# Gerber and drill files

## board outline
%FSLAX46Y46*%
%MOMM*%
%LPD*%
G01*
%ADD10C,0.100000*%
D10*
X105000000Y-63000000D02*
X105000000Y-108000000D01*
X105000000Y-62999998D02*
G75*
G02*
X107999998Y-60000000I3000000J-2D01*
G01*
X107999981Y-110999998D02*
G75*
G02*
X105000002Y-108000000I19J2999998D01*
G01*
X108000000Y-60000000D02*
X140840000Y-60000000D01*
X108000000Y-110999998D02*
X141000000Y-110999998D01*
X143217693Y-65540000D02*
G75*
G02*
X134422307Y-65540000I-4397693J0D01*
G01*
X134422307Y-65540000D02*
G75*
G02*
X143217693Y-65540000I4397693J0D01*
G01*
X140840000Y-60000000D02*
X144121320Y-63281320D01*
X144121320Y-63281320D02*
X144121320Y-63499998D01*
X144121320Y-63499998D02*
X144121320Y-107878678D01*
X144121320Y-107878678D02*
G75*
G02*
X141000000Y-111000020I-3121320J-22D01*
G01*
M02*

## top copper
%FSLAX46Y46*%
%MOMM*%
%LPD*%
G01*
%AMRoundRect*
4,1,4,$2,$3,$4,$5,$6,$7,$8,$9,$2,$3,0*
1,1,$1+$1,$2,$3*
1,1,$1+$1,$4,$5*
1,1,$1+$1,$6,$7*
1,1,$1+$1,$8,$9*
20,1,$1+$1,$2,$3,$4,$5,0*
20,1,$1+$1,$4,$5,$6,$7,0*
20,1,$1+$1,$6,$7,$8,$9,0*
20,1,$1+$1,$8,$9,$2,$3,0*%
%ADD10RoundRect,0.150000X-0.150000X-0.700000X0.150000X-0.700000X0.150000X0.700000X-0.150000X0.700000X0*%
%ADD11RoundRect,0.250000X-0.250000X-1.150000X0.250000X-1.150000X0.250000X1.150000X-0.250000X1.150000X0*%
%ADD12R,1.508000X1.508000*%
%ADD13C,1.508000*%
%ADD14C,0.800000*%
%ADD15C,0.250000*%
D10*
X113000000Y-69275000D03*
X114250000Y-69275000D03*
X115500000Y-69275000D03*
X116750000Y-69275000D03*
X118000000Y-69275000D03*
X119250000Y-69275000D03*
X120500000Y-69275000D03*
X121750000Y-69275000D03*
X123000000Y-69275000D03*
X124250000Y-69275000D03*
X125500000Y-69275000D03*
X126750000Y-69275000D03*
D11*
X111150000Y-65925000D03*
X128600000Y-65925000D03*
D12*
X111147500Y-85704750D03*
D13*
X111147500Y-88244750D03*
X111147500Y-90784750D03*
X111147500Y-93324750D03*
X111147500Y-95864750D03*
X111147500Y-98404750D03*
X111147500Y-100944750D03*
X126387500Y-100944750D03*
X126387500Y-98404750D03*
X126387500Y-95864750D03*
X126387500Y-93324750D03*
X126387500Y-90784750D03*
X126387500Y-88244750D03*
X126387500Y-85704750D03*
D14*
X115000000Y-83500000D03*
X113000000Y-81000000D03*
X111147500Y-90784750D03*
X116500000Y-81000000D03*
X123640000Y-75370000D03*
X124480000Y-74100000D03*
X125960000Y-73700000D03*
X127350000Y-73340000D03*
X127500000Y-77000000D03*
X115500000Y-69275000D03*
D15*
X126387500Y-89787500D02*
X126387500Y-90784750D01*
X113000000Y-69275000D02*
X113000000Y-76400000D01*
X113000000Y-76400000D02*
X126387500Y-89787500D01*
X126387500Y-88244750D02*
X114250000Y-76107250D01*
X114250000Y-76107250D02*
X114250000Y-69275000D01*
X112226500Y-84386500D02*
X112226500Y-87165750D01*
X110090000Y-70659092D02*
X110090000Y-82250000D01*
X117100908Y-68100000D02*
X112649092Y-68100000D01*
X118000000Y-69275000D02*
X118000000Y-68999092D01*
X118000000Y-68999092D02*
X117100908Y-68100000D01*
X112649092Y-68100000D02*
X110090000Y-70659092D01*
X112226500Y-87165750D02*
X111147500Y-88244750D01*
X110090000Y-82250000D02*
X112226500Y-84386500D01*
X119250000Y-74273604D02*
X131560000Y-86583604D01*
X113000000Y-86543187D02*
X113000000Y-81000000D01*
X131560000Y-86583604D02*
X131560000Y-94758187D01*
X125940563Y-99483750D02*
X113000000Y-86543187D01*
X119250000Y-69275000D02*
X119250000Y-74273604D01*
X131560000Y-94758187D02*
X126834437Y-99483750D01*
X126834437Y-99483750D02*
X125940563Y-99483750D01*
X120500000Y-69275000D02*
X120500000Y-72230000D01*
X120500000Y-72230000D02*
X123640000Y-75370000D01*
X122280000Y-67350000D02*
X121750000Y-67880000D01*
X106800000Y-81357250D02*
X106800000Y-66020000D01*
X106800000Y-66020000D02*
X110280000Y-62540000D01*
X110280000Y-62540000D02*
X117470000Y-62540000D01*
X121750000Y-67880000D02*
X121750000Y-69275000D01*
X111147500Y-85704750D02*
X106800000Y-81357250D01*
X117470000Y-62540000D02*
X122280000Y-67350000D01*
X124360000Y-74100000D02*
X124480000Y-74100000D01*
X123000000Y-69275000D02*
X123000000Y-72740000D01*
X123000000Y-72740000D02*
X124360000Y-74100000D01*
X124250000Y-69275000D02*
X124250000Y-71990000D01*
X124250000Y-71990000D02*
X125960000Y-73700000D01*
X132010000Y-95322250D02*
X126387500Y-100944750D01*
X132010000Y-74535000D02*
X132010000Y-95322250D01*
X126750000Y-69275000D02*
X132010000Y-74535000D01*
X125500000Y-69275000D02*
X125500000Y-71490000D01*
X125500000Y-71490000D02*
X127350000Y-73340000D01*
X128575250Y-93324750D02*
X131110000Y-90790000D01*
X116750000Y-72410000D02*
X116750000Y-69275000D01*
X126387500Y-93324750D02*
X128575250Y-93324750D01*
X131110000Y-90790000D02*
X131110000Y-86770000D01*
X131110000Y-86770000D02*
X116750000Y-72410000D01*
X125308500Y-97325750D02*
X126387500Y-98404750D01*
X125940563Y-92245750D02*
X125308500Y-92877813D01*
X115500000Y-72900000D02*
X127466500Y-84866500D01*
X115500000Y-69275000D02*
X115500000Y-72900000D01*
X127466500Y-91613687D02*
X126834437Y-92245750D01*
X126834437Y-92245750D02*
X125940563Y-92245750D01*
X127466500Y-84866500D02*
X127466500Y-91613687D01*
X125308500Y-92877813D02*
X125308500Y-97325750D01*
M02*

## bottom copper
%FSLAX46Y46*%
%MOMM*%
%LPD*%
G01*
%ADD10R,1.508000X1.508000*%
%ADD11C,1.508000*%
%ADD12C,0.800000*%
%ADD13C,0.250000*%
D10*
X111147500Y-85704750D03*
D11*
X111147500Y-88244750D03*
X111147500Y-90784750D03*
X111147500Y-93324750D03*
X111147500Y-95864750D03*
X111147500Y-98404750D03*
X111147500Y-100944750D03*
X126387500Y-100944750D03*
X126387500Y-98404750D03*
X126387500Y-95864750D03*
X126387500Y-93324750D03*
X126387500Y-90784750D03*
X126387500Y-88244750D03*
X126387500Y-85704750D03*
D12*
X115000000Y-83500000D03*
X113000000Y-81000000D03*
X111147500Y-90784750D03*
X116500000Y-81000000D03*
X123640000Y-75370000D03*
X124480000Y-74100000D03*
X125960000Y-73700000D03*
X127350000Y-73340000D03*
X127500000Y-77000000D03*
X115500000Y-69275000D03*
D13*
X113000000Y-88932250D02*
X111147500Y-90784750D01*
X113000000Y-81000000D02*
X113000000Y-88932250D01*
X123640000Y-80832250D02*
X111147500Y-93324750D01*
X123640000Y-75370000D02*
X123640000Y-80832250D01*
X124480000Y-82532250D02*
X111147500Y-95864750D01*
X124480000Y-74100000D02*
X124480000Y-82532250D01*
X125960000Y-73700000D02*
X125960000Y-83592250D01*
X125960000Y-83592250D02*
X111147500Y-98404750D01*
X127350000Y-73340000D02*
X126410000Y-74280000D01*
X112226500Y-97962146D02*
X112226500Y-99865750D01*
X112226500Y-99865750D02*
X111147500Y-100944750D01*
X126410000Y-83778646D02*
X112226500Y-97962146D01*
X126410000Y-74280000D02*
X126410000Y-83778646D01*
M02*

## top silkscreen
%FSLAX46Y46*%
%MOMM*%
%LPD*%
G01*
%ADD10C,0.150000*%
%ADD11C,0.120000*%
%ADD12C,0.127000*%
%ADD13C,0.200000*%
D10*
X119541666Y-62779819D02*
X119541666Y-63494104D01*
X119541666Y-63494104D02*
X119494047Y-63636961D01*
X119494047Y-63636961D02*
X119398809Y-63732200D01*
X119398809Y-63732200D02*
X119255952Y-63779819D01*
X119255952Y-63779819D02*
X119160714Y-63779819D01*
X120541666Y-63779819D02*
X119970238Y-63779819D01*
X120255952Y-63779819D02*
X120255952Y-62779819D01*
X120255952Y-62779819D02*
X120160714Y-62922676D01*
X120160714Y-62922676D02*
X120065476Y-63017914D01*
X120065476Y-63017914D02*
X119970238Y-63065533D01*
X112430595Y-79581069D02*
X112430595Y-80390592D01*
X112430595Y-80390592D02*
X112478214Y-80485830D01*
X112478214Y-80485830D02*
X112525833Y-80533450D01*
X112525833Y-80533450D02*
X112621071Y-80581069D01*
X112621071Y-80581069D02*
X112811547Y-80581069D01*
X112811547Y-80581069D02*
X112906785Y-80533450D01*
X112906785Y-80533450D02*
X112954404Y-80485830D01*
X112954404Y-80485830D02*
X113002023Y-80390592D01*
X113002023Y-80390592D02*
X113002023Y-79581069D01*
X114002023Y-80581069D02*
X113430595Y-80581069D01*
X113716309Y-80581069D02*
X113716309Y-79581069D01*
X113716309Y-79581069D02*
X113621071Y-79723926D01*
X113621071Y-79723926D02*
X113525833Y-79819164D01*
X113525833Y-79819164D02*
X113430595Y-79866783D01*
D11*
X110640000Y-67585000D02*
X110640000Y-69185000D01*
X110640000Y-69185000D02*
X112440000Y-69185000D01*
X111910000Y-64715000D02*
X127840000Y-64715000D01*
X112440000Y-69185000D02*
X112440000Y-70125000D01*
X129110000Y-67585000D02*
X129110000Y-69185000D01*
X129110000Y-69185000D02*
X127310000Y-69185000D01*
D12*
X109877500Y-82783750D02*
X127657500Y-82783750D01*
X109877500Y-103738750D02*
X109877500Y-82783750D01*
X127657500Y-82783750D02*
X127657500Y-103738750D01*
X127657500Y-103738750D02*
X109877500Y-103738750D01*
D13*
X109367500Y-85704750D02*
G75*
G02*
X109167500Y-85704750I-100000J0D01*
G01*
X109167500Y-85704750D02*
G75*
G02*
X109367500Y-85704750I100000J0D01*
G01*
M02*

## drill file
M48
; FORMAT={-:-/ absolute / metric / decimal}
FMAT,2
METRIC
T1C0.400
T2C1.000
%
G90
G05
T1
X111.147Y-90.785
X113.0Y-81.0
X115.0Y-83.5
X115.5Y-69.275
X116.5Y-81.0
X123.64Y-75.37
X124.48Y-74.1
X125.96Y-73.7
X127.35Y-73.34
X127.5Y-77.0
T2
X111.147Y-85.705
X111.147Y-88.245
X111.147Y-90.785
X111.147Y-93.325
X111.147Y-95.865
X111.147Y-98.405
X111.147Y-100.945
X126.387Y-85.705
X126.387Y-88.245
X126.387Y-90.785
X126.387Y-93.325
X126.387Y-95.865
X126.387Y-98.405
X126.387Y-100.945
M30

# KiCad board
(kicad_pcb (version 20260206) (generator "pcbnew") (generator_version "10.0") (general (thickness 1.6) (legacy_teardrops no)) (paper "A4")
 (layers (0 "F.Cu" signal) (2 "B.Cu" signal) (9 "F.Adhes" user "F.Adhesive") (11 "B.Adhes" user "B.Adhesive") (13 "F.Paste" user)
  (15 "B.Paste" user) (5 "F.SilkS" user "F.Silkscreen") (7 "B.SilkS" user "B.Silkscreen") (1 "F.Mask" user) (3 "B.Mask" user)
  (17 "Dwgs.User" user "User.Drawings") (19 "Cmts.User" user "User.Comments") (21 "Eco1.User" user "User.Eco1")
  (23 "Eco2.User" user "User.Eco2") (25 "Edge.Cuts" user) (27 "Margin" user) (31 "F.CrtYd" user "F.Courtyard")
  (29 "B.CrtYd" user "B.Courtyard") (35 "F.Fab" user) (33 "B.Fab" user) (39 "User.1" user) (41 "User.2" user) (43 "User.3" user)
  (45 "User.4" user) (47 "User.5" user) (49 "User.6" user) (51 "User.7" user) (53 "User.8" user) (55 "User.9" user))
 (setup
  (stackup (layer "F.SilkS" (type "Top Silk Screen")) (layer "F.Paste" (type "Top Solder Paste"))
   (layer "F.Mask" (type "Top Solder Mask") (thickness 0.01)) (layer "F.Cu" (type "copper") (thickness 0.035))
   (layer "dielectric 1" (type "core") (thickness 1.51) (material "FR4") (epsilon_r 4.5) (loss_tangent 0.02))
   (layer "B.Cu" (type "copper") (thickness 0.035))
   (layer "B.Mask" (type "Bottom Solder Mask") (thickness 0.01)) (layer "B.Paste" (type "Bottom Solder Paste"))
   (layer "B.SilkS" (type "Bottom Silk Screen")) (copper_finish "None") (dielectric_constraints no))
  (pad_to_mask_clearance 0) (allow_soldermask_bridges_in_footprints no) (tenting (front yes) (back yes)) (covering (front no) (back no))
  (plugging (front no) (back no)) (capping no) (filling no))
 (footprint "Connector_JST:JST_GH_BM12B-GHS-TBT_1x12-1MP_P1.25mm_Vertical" (layer "F.Cu") (at 119.875 67.325)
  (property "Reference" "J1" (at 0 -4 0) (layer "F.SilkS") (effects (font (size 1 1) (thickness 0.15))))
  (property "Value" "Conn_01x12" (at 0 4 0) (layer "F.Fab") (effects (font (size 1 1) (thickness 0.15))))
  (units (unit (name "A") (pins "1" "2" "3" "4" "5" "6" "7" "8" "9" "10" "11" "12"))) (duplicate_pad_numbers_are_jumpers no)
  (fp_line (start -9.235 0.26) (end -9.235 1.86) (stroke (width 0.12) (type solid)) (layer "F.SilkS"))
  (fp_line (start -9.235 1.86) (end -7.435 1.86) (stroke (width 0.12) (type solid)) (layer "F.SilkS"))
  (fp_line (start -7.965 -2.61) (end 7.965 -2.61) (stroke (width 0.12) (type solid)) (layer "F.SilkS"))
  (fp_line (start -7.435 1.86) (end -7.435 2.8) (stroke (width 0.12) (type solid)) (layer "F.SilkS"))
  (fp_line (start 9.235 0.26) (end 9.235 1.86) (stroke (width 0.12) (type solid)) (layer "F.SilkS"))
  (fp_line (start 9.235 1.86) (end 7.435 1.86) (stroke (width 0.12) (type solid)) (layer "F.SilkS"))
  (pad "1" smd roundrect (at -6.875 1.95) (size 0.6 1.7) (layers "F.Cu" "F.Mask" "F.Paste") (roundrect_rratio 0.25) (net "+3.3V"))
  (pad "2" smd roundrect (at -5.625 1.95) (size 0.6 1.7) (layers "F.Cu" "F.Mask" "F.Paste") (roundrect_rratio 0.25) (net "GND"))
  (pad "3" smd roundrect (at -4.375 1.95) (size 0.6 1.7) (layers "F.Cu" "F.Mask" "F.Paste") (roundrect_rratio 0.25) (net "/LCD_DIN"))
  (pad "4" smd roundrect (at -3.125 1.95) (size 0.6 1.7) (layers "F.Cu" "F.Mask" "F.Paste") (roundrect_rratio 0.25) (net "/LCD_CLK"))
  (pad "5" smd roundrect (at -1.875 1.95) (size 0.6 1.7) (layers "F.Cu" "F.Mask" "F.Paste") (roundrect_rratio 0.25) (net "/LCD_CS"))
  (pad "6" smd roundrect (at -0.625 1.95) (size 0.6 1.7) (layers "F.Cu" "F.Mask" "F.Paste") (roundrect_rratio 0.25) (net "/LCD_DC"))
  (pad "7" smd roundrect (at 0.625 1.95) (size 0.6 1.7) (layers "F.Cu" "F.Mask" "F.Paste") (roundrect_rratio 0.25) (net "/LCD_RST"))
  (pad "8" smd roundrect (at 1.875 1.95) (size 0.6 1.7) (layers "F.Cu" "F.Mask" "F.Paste") (roundrect_rratio 0.25) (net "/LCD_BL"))
  (pad "9" smd roundrect (at 3.125 1.95) (size 0.6 1.7) (layers "F.Cu" "F.Mask" "F.Paste") (roundrect_rratio 0.25) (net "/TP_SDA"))
  (pad "10" smd roundrect (at 4.375 1.95) (size 0.6 1.7) (layers "F.Cu" "F.Mask" "F.Paste") (roundrect_rratio 0.25) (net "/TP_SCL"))
  (pad "11" smd roundrect (at 5.625 1.95) (size 0.6 1.7) (layers "F.Cu" "F.Mask" "F.Paste") (roundrect_rratio 0.25) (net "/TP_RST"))
  (pad "12" smd roundrect (at 6.875 1.95) (size 0.6 1.7) (layers "F.Cu" "F.Mask" "F.Paste") (roundrect_rratio 0.25) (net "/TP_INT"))
  (pad "MP" smd roundrect (at -8.725 -1.4) (size 1 2.8) (layers "F.Cu" "F.Mask" "F.Paste") (roundrect_rratio 0.25))
  (pad "MP" smd roundrect (at 8.725 -1.4) (size 1 2.8) (layers "F.Cu" "F.Mask" "F.Paste") (roundrect_rratio 0.25)))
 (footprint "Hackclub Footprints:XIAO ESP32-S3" (layer "F.Cu") (at 118.7675 93.26125)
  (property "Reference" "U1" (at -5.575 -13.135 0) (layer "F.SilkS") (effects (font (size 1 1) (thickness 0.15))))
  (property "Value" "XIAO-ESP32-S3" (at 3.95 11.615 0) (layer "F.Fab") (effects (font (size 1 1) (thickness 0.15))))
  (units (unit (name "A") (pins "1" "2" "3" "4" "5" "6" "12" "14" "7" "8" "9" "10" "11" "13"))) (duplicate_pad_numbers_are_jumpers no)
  (fp_line (start -8.89 -10.4775) (end 8.89 -10.4775) (stroke (width 0.127) (type solid)) (layer "F.SilkS"))
  (fp_line (start -8.89 10.4775) (end -8.89 -10.4775) (stroke (width 0.127) (type solid)) (layer "F.SilkS"))
  (fp_line (start 8.89 -10.4775) (end 8.89 10.4775) (stroke (width 0.127) (type solid)) (layer "F.SilkS"))
  (fp_line (start 8.89 10.4775) (end -8.89 10.4775) (stroke (width 0.127) (type solid)) (layer "F.SilkS"))
  (fp_circle (center -9.5 -7.5565) (end -9.4 -7.5565) (stroke (width 0.2) (type solid)) (fill no) (layer "F.SilkS"))
  (pad "1" thru_hole rect (at -7.62 -7.5565) (size 1.508 1.508) (drill 1) (layers "*.Cu" "*.Mask") (remove_unused_layers no) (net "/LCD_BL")
   (solder_mask_margin 0.102))
  (pad "2" thru_hole circle (at -7.62 -5.0165) (size 1.508 1.508) (drill 1) (layers "*.Cu" "*.Mask") (remove_unused_layers no)
   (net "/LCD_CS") (solder_mask_margin 0.102))
  (pad "3" thru_hole circle (at -7.62 -2.4765) (size 1.508 1.508) (drill 1) (layers "*.Cu" "*.Mask") (remove_unused_layers no)
   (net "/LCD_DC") (solder_mask_margin 0.102))
  (pad "4" thru_hole circle (at -7.62 0.0635) (size 1.508 1.508) (drill 1) (layers "*.Cu" "*.Mask") (remove_unused_layers no)
   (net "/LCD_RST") (solder_mask_margin 0.102))
  (pad "5" thru_hole circle (at -7.62 2.6035) (size 1.508 1.508) (drill 1) (layers "*.Cu" "*.Mask") (remove_unused_layers no)
   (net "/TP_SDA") (solder_mask_margin 0.102))
  (pad "6" thru_hole circle (at -7.62 5.1435) (size 1.508 1.508) (drill 1) (layers "*.Cu" "*.Mask") (remove_unused_layers no)
   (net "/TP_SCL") (solder_mask_margin 0.102))
  (pad "7" thru_hole circle (at -7.62 7.6835) (size 1.508 1.508) (drill 1) (layers "*.Cu" "*.Mask") (remove_unused_layers no)
   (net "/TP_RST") (solder_mask_margin 0.102))
  (pad "8" thru_hole circle (at 7.62 7.6835) (size 1.508 1.508) (drill 1) (layers "*.Cu" "*.Mask") (remove_unused_layers no) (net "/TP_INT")
   (solder_mask_margin 0.102))
  (pad "9" thru_hole circle (at 7.62 5.1435) (size 1.508 1.508) (drill 1) (layers "*.Cu" "*.Mask") (remove_unused_layers no)
   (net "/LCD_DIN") (solder_mask_margin 0.102))
  (pad "10" thru_hole circle (at 7.62 2.6035) (size 1.508 1.508) (drill 1) (layers "*.Cu" "*.Mask") (remove_unused_layers no)
   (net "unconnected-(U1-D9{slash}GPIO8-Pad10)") (solder_mask_margin 0.102))
  (pad "11" thru_hole circle (at 7.62 0.0635) (size 1.508 1.508) (drill 1) (layers "*.Cu" "*.Mask") (remove_unused_layers no)
   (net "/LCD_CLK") (solder_mask_margin 0.102))
  (pad "12" thru_hole circle (at 7.62 -2.4765) (size 1.508 1.508) (drill 1) (layers "*.Cu" "*.Mask") (remove_unused_layers no) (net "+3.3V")
   (solder_mask_margin 0.102))
  (pad "13" thru_hole circle (at 7.62 -5.0165) (size 1.508 1.508) (drill 1) (layers "*.Cu" "*.Mask") (remove_unused_layers no) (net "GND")
   (solder_mask_margin 0.102))
  (pad "14" thru_hole circle (at 7.62 -7.5565) (size 1.508 1.508) (drill 1) (layers "*.Cu" "*.Mask") (remove_unused_layers no)
   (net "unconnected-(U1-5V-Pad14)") (solder_mask_margin 0.102)))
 (gr_line (start 105 63) (end 105 108) (stroke (width 0.1) (type default)) (layer "Edge.Cuts"))
 (gr_arc (start 105 62.999998) (mid 105.878679 60.878679) (end 107.999998 60) (stroke (width 0.1) (type default)) (layer "Edge.Cuts"))
 (gr_arc (start 107.999981 110.999998) (mid 105.878661 110.121319) (end 104.999982 108) (stroke (width 0.1) (type default))
  (layer "Edge.Cuts"))
 (gr_line (start 108 60) (end 140.84 60) (stroke (width 0.1) (type default)) (layer "Edge.Cuts"))
 (gr_line (start 108 110.999998) (end 141 110.999998) (stroke (width 0.1) (type default)) (layer "Edge.Cuts"))
 (gr_circle (center 138.82 65.54) (end 141.36 69.13) (stroke (width 0.1) (type default)) (fill no) (layer "Edge.Cuts"))
 (gr_line (start 140.84 60) (end 144.12132 63.28132) (stroke (width 0.1) (type default)) (layer "Edge.Cuts"))
 (gr_line (start 144.12132 63.28132) (end 144.12132 63.499998) (stroke (width 0.1) (type default)) (layer "Edge.Cuts"))
 (gr_line (start 144.12132 63.499998) (end 144.12132 107.878678) (stroke (width 0.1) (type default)) (layer "Edge.Cuts"))
 (gr_arc (start 144.12132 107.878678) (mid 143.207107 110.085785) (end 141 110.999998) (stroke (width 0.1) (type default))
  (layer "Edge.Cuts"))
 (segment (start 126.3875 89.7875) (end 126.3875 90.78475) (width 0.25) (layer "F.Cu") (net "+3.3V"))
 (segment (start 113 69.275) (end 113 76.4) (width 0.25) (layer "F.Cu") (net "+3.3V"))
 (segment (start 113 76.4) (end 126.3875 89.7875) (width 0.25) (layer "F.Cu") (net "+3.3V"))
 (segment (start 126.3875 88.24475) (end 114.25 76.10725) (width 0.25) (layer "F.Cu") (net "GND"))
 (segment (start 114.25 76.10725) (end 114.25 69.275) (width 0.25) (layer "F.Cu") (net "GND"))
 (segment (start 112.2265 84.3865) (end 112.2265 87.16575) (width 0.25) (layer "F.Cu") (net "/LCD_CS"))
 (segment (start 110.09 70.659092) (end 110.09 82.25) (width 0.25) (layer "F.Cu") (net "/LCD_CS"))
 (segment (start 117.100908 68.1) (end 112.649092 68.1) (width 0.25) (layer "F.Cu") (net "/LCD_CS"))
 (segment (start 118 69.275) (end 118 68.999092) (width 0.25) (layer "F.Cu") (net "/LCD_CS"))
 (segment (start 118 68.999092) (end 117.100908 68.1) (width 0.25) (layer "F.Cu") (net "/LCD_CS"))
 (segment (start 112.649092 68.1) (end 110.09 70.659092) (width 0.25) (layer "F.Cu") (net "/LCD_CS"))
 (segment (start 112.2265 87.16575) (end 111.1475 88.24475) (width 0.25) (layer "F.Cu") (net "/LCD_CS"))
 (segment (start 110.09 82.25) (end 112.2265 84.3865) (width 0.25) (layer "F.Cu") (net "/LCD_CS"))
 (via (at 115 83.5) (size 0.8) (drill 0.4) (layers "F.Cu" "B.Cu") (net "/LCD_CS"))
 (segment (start 119.25 74.273604) (end 131.56 86.583604) (width 0.25) (layer "F.Cu") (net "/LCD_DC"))
 (segment (start 113 86.543187) (end 113 81) (width 0.25) (layer "F.Cu") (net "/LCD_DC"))
 (segment (start 131.56 86.583604) (end 131.56 94.758187) (width 0.25) (layer "F.Cu") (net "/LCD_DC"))
 (segment (start 125.940563 99.48375) (end 113 86.543187) (width 0.25) (layer "F.Cu") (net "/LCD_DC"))
 (segment (start 119.25 69.275) (end 119.25 74.273604) (width 0.25) (layer "F.Cu") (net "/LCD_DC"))
 (segment (start 131.56 94.758187) (end 126.834437 99.48375) (width 0.25) (layer "F.Cu") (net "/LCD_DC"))
 (segment (start 126.834437 99.48375) (end 125.940563 99.48375) (width 0.25) (layer "F.Cu") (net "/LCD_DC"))
 (via (at 113 81) (size 0.8) (drill 0.4) (layers "F.Cu" "B.Cu") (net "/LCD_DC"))
 (via (at 111.1475 90.78475) (size 0.8) (drill 0.4) (layers "F.Cu" "B.Cu") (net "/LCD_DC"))
 (segment (start 113 88.93225) (end 111.1475 90.78475) (width 0.25) (layer "B.Cu") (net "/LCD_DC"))
 (segment (start 113 81) (end 113 88.93225) (width 0.25) (layer "B.Cu") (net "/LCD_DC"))
 (segment (start 120.5 69.275) (end 120.5 72.23) (width 0.25) (layer "F.Cu") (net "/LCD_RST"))
 (segment (start 120.5 72.23) (end 123.64 75.37) (width 0.25) (layer "F.Cu") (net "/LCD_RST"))
 (via (at 116.5 81) (size 0.8) (drill 0.4) (layers "F.Cu" "B.Cu") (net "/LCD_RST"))
 (via (at 123.64 75.37) (size 0.8) (drill 0.4) (layers "F.Cu" "B.Cu") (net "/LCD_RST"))
 (segment (start 123.64 80.83225) (end 111.1475 93.32475) (width 0.25) (layer "B.Cu") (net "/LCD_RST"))
 (segment (start 123.64 75.37) (end 123.64 80.83225) (width 0.25) (layer "B.Cu") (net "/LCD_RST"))
 (segment (start 122.28 67.35) (end 121.75 67.88) (width 0.25) (layer "F.Cu") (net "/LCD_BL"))
 (segment (start 106.8 81.35725) (end 106.8 66.02) (width 0.25) (layer "F.Cu") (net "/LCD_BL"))
 (segment (start 106.8 66.02) (end 110.28 62.54) (width 0.25) (layer "F.Cu") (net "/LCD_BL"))
 (segment (start 110.28 62.54) (end 117.47 62.54) (width 0.25) (layer "F.Cu") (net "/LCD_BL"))
 (segment (start 121.75 67.88) (end 121.75 69.275) (width 0.25) (layer "F.Cu") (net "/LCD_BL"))
 (segment (start 111.1475 85.70475) (end 106.8 81.35725) (width 0.25) (layer "F.Cu") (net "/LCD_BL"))
 (segment (start 117.47 62.54) (end 122.28 67.35) (width 0.25) (layer "F.Cu") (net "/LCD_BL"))
 (segment (start 124.36 74.1) (end 124.48 74.1) (width 0.25) (layer "F.Cu") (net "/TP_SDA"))
 (segment (start 123 69.275) (end 123 72.74) (width 0.25) (layer "F.Cu") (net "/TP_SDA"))
 (segment (start 123 72.74) (end 124.36 74.1) (width 0.25) (layer "F.Cu") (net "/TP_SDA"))
 (via (at 124.48 74.1) (size 0.8) (drill 0.4) (layers "F.Cu" "B.Cu") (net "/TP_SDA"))
 (segment (start 124.48 82.53225) (end 111.1475 95.86475) (width 0.25) (layer "B.Cu") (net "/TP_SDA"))
 (segment (start 124.48 74.1) (end 124.48 82.53225) (width 0.25) (layer "B.Cu") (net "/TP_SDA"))
 (segment (start 124.25 69.275) (end 124.25 71.99) (width 0.25) (layer "F.Cu") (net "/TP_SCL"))
 (segment (start 124.25 71.99) (end 125.96 73.7) (width 0.25) (layer "F.Cu") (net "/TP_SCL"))
 (via (at 125.96 73.7) (size 0.8) (drill 0.4) (layers "F.Cu" "B.Cu") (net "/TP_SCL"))
 (segment (start 125.96 73.7) (end 125.96 83.59225) (width 0.25) (layer "B.Cu") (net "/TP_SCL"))
 (segment (start 125.96 83.59225) (end 111.1475 98.40475) (width 0.25) (layer "B.Cu") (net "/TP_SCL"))
 (segment (start 132.01 95.32225) (end 126.3875 100.94475) (width 0.25) (layer "F.Cu") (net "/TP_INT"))
 (segment (start 132.01 74.535) (end 132.01 95.32225) (width 0.25) (layer "F.Cu") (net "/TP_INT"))
 (segment (start 126.75 69.275) (end 132.01 74.535) (width 0.25) (layer "F.Cu") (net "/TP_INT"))
 (segment (start 125.5 69.275) (end 125.5 71.49) (width 0.25) (layer "F.Cu") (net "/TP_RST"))
 (segment (start 125.5 71.49) (end 127.35 73.34) (width 0.25) (layer "F.Cu") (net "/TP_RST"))
 (via (at 127.35 73.34) (size 0.8) (drill 0.4) (layers "F.Cu" "B.Cu") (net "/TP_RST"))
 (segment (start 127.35 73.34) (end 126.41 74.28) (width 0.25) (layer "B.Cu") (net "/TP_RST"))
 (segment (start 112.2265 97.962146) (end 112.2265 99.86575) (width 0.25) (layer "B.Cu") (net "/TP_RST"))
 (segment (start 112.2265 99.86575) (end 111.1475 100.94475) (width 0.25) (layer "B.Cu") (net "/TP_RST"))
 (segment (start 126.41 83.778646) (end 112.2265 97.962146) (width 0.25) (layer "B.Cu") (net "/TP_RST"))
 (segment (start 126.41 74.28) (end 126.41 83.778646) (width 0.25) (layer "B.Cu") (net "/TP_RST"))
 (segment (start 128.57525 93.32475) (end 131.11 90.79) (width 0.25) (layer "F.Cu") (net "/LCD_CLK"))
 (segment (start 116.75 72.41) (end 116.75 69.275) (width 0.25) (layer "F.Cu") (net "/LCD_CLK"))
 (segment (start 126.3875 93.32475) (end 128.57525 93.32475) (width 0.25) (layer "F.Cu") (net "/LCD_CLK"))
 (segment (start 131.11 90.79) (end 131.11 86.77) (width 0.25) (layer "F.Cu") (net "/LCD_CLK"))
 (segment (start 131.11 86.77) (end 116.75 72.41) (width 0.25) (layer "F.Cu") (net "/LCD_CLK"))
 (segment (start 125.3085 97.32575) (end 126.3875 98.40475) (width 0.25) (layer "F.Cu") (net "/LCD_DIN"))
 (segment (start 125.940563 92.24575) (end 125.3085 92.877813) (width 0.25) (layer "F.Cu") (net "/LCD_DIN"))
 (segment (start 115.5 72.9) (end 127.4665 84.8665) (width 0.25) (layer "F.Cu") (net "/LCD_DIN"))
 (segment (start 115.5 69.275) (end 115.5 72.9) (width 0.25) (layer "F.Cu") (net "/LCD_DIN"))
 (segment (start 127.4665 91.613687) (end 126.834437 92.24575) (width 0.25) (layer "F.Cu") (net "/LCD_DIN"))
 (segment (start 126.834437 92.24575) (end 125.940563 92.24575) (width 0.25) (layer "F.Cu") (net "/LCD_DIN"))
 (segment (start 127.4665 84.8665) (end 127.4665 91.613687) (width 0.25) (layer "F.Cu") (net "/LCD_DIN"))
 (segment (start 125.3085 92.877813) (end 125.3085 97.32575) (width 0.25) (layer "F.Cu") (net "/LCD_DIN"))
 (via (at 127.5 77) (size 0.8) (drill 0.4) (layers "F.Cu" "B.Cu") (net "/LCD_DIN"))
 (via (at 115.5 69.275) (size 0.8) (drill 0.4) (layers "F.Cu" "B.Cu") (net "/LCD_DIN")))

